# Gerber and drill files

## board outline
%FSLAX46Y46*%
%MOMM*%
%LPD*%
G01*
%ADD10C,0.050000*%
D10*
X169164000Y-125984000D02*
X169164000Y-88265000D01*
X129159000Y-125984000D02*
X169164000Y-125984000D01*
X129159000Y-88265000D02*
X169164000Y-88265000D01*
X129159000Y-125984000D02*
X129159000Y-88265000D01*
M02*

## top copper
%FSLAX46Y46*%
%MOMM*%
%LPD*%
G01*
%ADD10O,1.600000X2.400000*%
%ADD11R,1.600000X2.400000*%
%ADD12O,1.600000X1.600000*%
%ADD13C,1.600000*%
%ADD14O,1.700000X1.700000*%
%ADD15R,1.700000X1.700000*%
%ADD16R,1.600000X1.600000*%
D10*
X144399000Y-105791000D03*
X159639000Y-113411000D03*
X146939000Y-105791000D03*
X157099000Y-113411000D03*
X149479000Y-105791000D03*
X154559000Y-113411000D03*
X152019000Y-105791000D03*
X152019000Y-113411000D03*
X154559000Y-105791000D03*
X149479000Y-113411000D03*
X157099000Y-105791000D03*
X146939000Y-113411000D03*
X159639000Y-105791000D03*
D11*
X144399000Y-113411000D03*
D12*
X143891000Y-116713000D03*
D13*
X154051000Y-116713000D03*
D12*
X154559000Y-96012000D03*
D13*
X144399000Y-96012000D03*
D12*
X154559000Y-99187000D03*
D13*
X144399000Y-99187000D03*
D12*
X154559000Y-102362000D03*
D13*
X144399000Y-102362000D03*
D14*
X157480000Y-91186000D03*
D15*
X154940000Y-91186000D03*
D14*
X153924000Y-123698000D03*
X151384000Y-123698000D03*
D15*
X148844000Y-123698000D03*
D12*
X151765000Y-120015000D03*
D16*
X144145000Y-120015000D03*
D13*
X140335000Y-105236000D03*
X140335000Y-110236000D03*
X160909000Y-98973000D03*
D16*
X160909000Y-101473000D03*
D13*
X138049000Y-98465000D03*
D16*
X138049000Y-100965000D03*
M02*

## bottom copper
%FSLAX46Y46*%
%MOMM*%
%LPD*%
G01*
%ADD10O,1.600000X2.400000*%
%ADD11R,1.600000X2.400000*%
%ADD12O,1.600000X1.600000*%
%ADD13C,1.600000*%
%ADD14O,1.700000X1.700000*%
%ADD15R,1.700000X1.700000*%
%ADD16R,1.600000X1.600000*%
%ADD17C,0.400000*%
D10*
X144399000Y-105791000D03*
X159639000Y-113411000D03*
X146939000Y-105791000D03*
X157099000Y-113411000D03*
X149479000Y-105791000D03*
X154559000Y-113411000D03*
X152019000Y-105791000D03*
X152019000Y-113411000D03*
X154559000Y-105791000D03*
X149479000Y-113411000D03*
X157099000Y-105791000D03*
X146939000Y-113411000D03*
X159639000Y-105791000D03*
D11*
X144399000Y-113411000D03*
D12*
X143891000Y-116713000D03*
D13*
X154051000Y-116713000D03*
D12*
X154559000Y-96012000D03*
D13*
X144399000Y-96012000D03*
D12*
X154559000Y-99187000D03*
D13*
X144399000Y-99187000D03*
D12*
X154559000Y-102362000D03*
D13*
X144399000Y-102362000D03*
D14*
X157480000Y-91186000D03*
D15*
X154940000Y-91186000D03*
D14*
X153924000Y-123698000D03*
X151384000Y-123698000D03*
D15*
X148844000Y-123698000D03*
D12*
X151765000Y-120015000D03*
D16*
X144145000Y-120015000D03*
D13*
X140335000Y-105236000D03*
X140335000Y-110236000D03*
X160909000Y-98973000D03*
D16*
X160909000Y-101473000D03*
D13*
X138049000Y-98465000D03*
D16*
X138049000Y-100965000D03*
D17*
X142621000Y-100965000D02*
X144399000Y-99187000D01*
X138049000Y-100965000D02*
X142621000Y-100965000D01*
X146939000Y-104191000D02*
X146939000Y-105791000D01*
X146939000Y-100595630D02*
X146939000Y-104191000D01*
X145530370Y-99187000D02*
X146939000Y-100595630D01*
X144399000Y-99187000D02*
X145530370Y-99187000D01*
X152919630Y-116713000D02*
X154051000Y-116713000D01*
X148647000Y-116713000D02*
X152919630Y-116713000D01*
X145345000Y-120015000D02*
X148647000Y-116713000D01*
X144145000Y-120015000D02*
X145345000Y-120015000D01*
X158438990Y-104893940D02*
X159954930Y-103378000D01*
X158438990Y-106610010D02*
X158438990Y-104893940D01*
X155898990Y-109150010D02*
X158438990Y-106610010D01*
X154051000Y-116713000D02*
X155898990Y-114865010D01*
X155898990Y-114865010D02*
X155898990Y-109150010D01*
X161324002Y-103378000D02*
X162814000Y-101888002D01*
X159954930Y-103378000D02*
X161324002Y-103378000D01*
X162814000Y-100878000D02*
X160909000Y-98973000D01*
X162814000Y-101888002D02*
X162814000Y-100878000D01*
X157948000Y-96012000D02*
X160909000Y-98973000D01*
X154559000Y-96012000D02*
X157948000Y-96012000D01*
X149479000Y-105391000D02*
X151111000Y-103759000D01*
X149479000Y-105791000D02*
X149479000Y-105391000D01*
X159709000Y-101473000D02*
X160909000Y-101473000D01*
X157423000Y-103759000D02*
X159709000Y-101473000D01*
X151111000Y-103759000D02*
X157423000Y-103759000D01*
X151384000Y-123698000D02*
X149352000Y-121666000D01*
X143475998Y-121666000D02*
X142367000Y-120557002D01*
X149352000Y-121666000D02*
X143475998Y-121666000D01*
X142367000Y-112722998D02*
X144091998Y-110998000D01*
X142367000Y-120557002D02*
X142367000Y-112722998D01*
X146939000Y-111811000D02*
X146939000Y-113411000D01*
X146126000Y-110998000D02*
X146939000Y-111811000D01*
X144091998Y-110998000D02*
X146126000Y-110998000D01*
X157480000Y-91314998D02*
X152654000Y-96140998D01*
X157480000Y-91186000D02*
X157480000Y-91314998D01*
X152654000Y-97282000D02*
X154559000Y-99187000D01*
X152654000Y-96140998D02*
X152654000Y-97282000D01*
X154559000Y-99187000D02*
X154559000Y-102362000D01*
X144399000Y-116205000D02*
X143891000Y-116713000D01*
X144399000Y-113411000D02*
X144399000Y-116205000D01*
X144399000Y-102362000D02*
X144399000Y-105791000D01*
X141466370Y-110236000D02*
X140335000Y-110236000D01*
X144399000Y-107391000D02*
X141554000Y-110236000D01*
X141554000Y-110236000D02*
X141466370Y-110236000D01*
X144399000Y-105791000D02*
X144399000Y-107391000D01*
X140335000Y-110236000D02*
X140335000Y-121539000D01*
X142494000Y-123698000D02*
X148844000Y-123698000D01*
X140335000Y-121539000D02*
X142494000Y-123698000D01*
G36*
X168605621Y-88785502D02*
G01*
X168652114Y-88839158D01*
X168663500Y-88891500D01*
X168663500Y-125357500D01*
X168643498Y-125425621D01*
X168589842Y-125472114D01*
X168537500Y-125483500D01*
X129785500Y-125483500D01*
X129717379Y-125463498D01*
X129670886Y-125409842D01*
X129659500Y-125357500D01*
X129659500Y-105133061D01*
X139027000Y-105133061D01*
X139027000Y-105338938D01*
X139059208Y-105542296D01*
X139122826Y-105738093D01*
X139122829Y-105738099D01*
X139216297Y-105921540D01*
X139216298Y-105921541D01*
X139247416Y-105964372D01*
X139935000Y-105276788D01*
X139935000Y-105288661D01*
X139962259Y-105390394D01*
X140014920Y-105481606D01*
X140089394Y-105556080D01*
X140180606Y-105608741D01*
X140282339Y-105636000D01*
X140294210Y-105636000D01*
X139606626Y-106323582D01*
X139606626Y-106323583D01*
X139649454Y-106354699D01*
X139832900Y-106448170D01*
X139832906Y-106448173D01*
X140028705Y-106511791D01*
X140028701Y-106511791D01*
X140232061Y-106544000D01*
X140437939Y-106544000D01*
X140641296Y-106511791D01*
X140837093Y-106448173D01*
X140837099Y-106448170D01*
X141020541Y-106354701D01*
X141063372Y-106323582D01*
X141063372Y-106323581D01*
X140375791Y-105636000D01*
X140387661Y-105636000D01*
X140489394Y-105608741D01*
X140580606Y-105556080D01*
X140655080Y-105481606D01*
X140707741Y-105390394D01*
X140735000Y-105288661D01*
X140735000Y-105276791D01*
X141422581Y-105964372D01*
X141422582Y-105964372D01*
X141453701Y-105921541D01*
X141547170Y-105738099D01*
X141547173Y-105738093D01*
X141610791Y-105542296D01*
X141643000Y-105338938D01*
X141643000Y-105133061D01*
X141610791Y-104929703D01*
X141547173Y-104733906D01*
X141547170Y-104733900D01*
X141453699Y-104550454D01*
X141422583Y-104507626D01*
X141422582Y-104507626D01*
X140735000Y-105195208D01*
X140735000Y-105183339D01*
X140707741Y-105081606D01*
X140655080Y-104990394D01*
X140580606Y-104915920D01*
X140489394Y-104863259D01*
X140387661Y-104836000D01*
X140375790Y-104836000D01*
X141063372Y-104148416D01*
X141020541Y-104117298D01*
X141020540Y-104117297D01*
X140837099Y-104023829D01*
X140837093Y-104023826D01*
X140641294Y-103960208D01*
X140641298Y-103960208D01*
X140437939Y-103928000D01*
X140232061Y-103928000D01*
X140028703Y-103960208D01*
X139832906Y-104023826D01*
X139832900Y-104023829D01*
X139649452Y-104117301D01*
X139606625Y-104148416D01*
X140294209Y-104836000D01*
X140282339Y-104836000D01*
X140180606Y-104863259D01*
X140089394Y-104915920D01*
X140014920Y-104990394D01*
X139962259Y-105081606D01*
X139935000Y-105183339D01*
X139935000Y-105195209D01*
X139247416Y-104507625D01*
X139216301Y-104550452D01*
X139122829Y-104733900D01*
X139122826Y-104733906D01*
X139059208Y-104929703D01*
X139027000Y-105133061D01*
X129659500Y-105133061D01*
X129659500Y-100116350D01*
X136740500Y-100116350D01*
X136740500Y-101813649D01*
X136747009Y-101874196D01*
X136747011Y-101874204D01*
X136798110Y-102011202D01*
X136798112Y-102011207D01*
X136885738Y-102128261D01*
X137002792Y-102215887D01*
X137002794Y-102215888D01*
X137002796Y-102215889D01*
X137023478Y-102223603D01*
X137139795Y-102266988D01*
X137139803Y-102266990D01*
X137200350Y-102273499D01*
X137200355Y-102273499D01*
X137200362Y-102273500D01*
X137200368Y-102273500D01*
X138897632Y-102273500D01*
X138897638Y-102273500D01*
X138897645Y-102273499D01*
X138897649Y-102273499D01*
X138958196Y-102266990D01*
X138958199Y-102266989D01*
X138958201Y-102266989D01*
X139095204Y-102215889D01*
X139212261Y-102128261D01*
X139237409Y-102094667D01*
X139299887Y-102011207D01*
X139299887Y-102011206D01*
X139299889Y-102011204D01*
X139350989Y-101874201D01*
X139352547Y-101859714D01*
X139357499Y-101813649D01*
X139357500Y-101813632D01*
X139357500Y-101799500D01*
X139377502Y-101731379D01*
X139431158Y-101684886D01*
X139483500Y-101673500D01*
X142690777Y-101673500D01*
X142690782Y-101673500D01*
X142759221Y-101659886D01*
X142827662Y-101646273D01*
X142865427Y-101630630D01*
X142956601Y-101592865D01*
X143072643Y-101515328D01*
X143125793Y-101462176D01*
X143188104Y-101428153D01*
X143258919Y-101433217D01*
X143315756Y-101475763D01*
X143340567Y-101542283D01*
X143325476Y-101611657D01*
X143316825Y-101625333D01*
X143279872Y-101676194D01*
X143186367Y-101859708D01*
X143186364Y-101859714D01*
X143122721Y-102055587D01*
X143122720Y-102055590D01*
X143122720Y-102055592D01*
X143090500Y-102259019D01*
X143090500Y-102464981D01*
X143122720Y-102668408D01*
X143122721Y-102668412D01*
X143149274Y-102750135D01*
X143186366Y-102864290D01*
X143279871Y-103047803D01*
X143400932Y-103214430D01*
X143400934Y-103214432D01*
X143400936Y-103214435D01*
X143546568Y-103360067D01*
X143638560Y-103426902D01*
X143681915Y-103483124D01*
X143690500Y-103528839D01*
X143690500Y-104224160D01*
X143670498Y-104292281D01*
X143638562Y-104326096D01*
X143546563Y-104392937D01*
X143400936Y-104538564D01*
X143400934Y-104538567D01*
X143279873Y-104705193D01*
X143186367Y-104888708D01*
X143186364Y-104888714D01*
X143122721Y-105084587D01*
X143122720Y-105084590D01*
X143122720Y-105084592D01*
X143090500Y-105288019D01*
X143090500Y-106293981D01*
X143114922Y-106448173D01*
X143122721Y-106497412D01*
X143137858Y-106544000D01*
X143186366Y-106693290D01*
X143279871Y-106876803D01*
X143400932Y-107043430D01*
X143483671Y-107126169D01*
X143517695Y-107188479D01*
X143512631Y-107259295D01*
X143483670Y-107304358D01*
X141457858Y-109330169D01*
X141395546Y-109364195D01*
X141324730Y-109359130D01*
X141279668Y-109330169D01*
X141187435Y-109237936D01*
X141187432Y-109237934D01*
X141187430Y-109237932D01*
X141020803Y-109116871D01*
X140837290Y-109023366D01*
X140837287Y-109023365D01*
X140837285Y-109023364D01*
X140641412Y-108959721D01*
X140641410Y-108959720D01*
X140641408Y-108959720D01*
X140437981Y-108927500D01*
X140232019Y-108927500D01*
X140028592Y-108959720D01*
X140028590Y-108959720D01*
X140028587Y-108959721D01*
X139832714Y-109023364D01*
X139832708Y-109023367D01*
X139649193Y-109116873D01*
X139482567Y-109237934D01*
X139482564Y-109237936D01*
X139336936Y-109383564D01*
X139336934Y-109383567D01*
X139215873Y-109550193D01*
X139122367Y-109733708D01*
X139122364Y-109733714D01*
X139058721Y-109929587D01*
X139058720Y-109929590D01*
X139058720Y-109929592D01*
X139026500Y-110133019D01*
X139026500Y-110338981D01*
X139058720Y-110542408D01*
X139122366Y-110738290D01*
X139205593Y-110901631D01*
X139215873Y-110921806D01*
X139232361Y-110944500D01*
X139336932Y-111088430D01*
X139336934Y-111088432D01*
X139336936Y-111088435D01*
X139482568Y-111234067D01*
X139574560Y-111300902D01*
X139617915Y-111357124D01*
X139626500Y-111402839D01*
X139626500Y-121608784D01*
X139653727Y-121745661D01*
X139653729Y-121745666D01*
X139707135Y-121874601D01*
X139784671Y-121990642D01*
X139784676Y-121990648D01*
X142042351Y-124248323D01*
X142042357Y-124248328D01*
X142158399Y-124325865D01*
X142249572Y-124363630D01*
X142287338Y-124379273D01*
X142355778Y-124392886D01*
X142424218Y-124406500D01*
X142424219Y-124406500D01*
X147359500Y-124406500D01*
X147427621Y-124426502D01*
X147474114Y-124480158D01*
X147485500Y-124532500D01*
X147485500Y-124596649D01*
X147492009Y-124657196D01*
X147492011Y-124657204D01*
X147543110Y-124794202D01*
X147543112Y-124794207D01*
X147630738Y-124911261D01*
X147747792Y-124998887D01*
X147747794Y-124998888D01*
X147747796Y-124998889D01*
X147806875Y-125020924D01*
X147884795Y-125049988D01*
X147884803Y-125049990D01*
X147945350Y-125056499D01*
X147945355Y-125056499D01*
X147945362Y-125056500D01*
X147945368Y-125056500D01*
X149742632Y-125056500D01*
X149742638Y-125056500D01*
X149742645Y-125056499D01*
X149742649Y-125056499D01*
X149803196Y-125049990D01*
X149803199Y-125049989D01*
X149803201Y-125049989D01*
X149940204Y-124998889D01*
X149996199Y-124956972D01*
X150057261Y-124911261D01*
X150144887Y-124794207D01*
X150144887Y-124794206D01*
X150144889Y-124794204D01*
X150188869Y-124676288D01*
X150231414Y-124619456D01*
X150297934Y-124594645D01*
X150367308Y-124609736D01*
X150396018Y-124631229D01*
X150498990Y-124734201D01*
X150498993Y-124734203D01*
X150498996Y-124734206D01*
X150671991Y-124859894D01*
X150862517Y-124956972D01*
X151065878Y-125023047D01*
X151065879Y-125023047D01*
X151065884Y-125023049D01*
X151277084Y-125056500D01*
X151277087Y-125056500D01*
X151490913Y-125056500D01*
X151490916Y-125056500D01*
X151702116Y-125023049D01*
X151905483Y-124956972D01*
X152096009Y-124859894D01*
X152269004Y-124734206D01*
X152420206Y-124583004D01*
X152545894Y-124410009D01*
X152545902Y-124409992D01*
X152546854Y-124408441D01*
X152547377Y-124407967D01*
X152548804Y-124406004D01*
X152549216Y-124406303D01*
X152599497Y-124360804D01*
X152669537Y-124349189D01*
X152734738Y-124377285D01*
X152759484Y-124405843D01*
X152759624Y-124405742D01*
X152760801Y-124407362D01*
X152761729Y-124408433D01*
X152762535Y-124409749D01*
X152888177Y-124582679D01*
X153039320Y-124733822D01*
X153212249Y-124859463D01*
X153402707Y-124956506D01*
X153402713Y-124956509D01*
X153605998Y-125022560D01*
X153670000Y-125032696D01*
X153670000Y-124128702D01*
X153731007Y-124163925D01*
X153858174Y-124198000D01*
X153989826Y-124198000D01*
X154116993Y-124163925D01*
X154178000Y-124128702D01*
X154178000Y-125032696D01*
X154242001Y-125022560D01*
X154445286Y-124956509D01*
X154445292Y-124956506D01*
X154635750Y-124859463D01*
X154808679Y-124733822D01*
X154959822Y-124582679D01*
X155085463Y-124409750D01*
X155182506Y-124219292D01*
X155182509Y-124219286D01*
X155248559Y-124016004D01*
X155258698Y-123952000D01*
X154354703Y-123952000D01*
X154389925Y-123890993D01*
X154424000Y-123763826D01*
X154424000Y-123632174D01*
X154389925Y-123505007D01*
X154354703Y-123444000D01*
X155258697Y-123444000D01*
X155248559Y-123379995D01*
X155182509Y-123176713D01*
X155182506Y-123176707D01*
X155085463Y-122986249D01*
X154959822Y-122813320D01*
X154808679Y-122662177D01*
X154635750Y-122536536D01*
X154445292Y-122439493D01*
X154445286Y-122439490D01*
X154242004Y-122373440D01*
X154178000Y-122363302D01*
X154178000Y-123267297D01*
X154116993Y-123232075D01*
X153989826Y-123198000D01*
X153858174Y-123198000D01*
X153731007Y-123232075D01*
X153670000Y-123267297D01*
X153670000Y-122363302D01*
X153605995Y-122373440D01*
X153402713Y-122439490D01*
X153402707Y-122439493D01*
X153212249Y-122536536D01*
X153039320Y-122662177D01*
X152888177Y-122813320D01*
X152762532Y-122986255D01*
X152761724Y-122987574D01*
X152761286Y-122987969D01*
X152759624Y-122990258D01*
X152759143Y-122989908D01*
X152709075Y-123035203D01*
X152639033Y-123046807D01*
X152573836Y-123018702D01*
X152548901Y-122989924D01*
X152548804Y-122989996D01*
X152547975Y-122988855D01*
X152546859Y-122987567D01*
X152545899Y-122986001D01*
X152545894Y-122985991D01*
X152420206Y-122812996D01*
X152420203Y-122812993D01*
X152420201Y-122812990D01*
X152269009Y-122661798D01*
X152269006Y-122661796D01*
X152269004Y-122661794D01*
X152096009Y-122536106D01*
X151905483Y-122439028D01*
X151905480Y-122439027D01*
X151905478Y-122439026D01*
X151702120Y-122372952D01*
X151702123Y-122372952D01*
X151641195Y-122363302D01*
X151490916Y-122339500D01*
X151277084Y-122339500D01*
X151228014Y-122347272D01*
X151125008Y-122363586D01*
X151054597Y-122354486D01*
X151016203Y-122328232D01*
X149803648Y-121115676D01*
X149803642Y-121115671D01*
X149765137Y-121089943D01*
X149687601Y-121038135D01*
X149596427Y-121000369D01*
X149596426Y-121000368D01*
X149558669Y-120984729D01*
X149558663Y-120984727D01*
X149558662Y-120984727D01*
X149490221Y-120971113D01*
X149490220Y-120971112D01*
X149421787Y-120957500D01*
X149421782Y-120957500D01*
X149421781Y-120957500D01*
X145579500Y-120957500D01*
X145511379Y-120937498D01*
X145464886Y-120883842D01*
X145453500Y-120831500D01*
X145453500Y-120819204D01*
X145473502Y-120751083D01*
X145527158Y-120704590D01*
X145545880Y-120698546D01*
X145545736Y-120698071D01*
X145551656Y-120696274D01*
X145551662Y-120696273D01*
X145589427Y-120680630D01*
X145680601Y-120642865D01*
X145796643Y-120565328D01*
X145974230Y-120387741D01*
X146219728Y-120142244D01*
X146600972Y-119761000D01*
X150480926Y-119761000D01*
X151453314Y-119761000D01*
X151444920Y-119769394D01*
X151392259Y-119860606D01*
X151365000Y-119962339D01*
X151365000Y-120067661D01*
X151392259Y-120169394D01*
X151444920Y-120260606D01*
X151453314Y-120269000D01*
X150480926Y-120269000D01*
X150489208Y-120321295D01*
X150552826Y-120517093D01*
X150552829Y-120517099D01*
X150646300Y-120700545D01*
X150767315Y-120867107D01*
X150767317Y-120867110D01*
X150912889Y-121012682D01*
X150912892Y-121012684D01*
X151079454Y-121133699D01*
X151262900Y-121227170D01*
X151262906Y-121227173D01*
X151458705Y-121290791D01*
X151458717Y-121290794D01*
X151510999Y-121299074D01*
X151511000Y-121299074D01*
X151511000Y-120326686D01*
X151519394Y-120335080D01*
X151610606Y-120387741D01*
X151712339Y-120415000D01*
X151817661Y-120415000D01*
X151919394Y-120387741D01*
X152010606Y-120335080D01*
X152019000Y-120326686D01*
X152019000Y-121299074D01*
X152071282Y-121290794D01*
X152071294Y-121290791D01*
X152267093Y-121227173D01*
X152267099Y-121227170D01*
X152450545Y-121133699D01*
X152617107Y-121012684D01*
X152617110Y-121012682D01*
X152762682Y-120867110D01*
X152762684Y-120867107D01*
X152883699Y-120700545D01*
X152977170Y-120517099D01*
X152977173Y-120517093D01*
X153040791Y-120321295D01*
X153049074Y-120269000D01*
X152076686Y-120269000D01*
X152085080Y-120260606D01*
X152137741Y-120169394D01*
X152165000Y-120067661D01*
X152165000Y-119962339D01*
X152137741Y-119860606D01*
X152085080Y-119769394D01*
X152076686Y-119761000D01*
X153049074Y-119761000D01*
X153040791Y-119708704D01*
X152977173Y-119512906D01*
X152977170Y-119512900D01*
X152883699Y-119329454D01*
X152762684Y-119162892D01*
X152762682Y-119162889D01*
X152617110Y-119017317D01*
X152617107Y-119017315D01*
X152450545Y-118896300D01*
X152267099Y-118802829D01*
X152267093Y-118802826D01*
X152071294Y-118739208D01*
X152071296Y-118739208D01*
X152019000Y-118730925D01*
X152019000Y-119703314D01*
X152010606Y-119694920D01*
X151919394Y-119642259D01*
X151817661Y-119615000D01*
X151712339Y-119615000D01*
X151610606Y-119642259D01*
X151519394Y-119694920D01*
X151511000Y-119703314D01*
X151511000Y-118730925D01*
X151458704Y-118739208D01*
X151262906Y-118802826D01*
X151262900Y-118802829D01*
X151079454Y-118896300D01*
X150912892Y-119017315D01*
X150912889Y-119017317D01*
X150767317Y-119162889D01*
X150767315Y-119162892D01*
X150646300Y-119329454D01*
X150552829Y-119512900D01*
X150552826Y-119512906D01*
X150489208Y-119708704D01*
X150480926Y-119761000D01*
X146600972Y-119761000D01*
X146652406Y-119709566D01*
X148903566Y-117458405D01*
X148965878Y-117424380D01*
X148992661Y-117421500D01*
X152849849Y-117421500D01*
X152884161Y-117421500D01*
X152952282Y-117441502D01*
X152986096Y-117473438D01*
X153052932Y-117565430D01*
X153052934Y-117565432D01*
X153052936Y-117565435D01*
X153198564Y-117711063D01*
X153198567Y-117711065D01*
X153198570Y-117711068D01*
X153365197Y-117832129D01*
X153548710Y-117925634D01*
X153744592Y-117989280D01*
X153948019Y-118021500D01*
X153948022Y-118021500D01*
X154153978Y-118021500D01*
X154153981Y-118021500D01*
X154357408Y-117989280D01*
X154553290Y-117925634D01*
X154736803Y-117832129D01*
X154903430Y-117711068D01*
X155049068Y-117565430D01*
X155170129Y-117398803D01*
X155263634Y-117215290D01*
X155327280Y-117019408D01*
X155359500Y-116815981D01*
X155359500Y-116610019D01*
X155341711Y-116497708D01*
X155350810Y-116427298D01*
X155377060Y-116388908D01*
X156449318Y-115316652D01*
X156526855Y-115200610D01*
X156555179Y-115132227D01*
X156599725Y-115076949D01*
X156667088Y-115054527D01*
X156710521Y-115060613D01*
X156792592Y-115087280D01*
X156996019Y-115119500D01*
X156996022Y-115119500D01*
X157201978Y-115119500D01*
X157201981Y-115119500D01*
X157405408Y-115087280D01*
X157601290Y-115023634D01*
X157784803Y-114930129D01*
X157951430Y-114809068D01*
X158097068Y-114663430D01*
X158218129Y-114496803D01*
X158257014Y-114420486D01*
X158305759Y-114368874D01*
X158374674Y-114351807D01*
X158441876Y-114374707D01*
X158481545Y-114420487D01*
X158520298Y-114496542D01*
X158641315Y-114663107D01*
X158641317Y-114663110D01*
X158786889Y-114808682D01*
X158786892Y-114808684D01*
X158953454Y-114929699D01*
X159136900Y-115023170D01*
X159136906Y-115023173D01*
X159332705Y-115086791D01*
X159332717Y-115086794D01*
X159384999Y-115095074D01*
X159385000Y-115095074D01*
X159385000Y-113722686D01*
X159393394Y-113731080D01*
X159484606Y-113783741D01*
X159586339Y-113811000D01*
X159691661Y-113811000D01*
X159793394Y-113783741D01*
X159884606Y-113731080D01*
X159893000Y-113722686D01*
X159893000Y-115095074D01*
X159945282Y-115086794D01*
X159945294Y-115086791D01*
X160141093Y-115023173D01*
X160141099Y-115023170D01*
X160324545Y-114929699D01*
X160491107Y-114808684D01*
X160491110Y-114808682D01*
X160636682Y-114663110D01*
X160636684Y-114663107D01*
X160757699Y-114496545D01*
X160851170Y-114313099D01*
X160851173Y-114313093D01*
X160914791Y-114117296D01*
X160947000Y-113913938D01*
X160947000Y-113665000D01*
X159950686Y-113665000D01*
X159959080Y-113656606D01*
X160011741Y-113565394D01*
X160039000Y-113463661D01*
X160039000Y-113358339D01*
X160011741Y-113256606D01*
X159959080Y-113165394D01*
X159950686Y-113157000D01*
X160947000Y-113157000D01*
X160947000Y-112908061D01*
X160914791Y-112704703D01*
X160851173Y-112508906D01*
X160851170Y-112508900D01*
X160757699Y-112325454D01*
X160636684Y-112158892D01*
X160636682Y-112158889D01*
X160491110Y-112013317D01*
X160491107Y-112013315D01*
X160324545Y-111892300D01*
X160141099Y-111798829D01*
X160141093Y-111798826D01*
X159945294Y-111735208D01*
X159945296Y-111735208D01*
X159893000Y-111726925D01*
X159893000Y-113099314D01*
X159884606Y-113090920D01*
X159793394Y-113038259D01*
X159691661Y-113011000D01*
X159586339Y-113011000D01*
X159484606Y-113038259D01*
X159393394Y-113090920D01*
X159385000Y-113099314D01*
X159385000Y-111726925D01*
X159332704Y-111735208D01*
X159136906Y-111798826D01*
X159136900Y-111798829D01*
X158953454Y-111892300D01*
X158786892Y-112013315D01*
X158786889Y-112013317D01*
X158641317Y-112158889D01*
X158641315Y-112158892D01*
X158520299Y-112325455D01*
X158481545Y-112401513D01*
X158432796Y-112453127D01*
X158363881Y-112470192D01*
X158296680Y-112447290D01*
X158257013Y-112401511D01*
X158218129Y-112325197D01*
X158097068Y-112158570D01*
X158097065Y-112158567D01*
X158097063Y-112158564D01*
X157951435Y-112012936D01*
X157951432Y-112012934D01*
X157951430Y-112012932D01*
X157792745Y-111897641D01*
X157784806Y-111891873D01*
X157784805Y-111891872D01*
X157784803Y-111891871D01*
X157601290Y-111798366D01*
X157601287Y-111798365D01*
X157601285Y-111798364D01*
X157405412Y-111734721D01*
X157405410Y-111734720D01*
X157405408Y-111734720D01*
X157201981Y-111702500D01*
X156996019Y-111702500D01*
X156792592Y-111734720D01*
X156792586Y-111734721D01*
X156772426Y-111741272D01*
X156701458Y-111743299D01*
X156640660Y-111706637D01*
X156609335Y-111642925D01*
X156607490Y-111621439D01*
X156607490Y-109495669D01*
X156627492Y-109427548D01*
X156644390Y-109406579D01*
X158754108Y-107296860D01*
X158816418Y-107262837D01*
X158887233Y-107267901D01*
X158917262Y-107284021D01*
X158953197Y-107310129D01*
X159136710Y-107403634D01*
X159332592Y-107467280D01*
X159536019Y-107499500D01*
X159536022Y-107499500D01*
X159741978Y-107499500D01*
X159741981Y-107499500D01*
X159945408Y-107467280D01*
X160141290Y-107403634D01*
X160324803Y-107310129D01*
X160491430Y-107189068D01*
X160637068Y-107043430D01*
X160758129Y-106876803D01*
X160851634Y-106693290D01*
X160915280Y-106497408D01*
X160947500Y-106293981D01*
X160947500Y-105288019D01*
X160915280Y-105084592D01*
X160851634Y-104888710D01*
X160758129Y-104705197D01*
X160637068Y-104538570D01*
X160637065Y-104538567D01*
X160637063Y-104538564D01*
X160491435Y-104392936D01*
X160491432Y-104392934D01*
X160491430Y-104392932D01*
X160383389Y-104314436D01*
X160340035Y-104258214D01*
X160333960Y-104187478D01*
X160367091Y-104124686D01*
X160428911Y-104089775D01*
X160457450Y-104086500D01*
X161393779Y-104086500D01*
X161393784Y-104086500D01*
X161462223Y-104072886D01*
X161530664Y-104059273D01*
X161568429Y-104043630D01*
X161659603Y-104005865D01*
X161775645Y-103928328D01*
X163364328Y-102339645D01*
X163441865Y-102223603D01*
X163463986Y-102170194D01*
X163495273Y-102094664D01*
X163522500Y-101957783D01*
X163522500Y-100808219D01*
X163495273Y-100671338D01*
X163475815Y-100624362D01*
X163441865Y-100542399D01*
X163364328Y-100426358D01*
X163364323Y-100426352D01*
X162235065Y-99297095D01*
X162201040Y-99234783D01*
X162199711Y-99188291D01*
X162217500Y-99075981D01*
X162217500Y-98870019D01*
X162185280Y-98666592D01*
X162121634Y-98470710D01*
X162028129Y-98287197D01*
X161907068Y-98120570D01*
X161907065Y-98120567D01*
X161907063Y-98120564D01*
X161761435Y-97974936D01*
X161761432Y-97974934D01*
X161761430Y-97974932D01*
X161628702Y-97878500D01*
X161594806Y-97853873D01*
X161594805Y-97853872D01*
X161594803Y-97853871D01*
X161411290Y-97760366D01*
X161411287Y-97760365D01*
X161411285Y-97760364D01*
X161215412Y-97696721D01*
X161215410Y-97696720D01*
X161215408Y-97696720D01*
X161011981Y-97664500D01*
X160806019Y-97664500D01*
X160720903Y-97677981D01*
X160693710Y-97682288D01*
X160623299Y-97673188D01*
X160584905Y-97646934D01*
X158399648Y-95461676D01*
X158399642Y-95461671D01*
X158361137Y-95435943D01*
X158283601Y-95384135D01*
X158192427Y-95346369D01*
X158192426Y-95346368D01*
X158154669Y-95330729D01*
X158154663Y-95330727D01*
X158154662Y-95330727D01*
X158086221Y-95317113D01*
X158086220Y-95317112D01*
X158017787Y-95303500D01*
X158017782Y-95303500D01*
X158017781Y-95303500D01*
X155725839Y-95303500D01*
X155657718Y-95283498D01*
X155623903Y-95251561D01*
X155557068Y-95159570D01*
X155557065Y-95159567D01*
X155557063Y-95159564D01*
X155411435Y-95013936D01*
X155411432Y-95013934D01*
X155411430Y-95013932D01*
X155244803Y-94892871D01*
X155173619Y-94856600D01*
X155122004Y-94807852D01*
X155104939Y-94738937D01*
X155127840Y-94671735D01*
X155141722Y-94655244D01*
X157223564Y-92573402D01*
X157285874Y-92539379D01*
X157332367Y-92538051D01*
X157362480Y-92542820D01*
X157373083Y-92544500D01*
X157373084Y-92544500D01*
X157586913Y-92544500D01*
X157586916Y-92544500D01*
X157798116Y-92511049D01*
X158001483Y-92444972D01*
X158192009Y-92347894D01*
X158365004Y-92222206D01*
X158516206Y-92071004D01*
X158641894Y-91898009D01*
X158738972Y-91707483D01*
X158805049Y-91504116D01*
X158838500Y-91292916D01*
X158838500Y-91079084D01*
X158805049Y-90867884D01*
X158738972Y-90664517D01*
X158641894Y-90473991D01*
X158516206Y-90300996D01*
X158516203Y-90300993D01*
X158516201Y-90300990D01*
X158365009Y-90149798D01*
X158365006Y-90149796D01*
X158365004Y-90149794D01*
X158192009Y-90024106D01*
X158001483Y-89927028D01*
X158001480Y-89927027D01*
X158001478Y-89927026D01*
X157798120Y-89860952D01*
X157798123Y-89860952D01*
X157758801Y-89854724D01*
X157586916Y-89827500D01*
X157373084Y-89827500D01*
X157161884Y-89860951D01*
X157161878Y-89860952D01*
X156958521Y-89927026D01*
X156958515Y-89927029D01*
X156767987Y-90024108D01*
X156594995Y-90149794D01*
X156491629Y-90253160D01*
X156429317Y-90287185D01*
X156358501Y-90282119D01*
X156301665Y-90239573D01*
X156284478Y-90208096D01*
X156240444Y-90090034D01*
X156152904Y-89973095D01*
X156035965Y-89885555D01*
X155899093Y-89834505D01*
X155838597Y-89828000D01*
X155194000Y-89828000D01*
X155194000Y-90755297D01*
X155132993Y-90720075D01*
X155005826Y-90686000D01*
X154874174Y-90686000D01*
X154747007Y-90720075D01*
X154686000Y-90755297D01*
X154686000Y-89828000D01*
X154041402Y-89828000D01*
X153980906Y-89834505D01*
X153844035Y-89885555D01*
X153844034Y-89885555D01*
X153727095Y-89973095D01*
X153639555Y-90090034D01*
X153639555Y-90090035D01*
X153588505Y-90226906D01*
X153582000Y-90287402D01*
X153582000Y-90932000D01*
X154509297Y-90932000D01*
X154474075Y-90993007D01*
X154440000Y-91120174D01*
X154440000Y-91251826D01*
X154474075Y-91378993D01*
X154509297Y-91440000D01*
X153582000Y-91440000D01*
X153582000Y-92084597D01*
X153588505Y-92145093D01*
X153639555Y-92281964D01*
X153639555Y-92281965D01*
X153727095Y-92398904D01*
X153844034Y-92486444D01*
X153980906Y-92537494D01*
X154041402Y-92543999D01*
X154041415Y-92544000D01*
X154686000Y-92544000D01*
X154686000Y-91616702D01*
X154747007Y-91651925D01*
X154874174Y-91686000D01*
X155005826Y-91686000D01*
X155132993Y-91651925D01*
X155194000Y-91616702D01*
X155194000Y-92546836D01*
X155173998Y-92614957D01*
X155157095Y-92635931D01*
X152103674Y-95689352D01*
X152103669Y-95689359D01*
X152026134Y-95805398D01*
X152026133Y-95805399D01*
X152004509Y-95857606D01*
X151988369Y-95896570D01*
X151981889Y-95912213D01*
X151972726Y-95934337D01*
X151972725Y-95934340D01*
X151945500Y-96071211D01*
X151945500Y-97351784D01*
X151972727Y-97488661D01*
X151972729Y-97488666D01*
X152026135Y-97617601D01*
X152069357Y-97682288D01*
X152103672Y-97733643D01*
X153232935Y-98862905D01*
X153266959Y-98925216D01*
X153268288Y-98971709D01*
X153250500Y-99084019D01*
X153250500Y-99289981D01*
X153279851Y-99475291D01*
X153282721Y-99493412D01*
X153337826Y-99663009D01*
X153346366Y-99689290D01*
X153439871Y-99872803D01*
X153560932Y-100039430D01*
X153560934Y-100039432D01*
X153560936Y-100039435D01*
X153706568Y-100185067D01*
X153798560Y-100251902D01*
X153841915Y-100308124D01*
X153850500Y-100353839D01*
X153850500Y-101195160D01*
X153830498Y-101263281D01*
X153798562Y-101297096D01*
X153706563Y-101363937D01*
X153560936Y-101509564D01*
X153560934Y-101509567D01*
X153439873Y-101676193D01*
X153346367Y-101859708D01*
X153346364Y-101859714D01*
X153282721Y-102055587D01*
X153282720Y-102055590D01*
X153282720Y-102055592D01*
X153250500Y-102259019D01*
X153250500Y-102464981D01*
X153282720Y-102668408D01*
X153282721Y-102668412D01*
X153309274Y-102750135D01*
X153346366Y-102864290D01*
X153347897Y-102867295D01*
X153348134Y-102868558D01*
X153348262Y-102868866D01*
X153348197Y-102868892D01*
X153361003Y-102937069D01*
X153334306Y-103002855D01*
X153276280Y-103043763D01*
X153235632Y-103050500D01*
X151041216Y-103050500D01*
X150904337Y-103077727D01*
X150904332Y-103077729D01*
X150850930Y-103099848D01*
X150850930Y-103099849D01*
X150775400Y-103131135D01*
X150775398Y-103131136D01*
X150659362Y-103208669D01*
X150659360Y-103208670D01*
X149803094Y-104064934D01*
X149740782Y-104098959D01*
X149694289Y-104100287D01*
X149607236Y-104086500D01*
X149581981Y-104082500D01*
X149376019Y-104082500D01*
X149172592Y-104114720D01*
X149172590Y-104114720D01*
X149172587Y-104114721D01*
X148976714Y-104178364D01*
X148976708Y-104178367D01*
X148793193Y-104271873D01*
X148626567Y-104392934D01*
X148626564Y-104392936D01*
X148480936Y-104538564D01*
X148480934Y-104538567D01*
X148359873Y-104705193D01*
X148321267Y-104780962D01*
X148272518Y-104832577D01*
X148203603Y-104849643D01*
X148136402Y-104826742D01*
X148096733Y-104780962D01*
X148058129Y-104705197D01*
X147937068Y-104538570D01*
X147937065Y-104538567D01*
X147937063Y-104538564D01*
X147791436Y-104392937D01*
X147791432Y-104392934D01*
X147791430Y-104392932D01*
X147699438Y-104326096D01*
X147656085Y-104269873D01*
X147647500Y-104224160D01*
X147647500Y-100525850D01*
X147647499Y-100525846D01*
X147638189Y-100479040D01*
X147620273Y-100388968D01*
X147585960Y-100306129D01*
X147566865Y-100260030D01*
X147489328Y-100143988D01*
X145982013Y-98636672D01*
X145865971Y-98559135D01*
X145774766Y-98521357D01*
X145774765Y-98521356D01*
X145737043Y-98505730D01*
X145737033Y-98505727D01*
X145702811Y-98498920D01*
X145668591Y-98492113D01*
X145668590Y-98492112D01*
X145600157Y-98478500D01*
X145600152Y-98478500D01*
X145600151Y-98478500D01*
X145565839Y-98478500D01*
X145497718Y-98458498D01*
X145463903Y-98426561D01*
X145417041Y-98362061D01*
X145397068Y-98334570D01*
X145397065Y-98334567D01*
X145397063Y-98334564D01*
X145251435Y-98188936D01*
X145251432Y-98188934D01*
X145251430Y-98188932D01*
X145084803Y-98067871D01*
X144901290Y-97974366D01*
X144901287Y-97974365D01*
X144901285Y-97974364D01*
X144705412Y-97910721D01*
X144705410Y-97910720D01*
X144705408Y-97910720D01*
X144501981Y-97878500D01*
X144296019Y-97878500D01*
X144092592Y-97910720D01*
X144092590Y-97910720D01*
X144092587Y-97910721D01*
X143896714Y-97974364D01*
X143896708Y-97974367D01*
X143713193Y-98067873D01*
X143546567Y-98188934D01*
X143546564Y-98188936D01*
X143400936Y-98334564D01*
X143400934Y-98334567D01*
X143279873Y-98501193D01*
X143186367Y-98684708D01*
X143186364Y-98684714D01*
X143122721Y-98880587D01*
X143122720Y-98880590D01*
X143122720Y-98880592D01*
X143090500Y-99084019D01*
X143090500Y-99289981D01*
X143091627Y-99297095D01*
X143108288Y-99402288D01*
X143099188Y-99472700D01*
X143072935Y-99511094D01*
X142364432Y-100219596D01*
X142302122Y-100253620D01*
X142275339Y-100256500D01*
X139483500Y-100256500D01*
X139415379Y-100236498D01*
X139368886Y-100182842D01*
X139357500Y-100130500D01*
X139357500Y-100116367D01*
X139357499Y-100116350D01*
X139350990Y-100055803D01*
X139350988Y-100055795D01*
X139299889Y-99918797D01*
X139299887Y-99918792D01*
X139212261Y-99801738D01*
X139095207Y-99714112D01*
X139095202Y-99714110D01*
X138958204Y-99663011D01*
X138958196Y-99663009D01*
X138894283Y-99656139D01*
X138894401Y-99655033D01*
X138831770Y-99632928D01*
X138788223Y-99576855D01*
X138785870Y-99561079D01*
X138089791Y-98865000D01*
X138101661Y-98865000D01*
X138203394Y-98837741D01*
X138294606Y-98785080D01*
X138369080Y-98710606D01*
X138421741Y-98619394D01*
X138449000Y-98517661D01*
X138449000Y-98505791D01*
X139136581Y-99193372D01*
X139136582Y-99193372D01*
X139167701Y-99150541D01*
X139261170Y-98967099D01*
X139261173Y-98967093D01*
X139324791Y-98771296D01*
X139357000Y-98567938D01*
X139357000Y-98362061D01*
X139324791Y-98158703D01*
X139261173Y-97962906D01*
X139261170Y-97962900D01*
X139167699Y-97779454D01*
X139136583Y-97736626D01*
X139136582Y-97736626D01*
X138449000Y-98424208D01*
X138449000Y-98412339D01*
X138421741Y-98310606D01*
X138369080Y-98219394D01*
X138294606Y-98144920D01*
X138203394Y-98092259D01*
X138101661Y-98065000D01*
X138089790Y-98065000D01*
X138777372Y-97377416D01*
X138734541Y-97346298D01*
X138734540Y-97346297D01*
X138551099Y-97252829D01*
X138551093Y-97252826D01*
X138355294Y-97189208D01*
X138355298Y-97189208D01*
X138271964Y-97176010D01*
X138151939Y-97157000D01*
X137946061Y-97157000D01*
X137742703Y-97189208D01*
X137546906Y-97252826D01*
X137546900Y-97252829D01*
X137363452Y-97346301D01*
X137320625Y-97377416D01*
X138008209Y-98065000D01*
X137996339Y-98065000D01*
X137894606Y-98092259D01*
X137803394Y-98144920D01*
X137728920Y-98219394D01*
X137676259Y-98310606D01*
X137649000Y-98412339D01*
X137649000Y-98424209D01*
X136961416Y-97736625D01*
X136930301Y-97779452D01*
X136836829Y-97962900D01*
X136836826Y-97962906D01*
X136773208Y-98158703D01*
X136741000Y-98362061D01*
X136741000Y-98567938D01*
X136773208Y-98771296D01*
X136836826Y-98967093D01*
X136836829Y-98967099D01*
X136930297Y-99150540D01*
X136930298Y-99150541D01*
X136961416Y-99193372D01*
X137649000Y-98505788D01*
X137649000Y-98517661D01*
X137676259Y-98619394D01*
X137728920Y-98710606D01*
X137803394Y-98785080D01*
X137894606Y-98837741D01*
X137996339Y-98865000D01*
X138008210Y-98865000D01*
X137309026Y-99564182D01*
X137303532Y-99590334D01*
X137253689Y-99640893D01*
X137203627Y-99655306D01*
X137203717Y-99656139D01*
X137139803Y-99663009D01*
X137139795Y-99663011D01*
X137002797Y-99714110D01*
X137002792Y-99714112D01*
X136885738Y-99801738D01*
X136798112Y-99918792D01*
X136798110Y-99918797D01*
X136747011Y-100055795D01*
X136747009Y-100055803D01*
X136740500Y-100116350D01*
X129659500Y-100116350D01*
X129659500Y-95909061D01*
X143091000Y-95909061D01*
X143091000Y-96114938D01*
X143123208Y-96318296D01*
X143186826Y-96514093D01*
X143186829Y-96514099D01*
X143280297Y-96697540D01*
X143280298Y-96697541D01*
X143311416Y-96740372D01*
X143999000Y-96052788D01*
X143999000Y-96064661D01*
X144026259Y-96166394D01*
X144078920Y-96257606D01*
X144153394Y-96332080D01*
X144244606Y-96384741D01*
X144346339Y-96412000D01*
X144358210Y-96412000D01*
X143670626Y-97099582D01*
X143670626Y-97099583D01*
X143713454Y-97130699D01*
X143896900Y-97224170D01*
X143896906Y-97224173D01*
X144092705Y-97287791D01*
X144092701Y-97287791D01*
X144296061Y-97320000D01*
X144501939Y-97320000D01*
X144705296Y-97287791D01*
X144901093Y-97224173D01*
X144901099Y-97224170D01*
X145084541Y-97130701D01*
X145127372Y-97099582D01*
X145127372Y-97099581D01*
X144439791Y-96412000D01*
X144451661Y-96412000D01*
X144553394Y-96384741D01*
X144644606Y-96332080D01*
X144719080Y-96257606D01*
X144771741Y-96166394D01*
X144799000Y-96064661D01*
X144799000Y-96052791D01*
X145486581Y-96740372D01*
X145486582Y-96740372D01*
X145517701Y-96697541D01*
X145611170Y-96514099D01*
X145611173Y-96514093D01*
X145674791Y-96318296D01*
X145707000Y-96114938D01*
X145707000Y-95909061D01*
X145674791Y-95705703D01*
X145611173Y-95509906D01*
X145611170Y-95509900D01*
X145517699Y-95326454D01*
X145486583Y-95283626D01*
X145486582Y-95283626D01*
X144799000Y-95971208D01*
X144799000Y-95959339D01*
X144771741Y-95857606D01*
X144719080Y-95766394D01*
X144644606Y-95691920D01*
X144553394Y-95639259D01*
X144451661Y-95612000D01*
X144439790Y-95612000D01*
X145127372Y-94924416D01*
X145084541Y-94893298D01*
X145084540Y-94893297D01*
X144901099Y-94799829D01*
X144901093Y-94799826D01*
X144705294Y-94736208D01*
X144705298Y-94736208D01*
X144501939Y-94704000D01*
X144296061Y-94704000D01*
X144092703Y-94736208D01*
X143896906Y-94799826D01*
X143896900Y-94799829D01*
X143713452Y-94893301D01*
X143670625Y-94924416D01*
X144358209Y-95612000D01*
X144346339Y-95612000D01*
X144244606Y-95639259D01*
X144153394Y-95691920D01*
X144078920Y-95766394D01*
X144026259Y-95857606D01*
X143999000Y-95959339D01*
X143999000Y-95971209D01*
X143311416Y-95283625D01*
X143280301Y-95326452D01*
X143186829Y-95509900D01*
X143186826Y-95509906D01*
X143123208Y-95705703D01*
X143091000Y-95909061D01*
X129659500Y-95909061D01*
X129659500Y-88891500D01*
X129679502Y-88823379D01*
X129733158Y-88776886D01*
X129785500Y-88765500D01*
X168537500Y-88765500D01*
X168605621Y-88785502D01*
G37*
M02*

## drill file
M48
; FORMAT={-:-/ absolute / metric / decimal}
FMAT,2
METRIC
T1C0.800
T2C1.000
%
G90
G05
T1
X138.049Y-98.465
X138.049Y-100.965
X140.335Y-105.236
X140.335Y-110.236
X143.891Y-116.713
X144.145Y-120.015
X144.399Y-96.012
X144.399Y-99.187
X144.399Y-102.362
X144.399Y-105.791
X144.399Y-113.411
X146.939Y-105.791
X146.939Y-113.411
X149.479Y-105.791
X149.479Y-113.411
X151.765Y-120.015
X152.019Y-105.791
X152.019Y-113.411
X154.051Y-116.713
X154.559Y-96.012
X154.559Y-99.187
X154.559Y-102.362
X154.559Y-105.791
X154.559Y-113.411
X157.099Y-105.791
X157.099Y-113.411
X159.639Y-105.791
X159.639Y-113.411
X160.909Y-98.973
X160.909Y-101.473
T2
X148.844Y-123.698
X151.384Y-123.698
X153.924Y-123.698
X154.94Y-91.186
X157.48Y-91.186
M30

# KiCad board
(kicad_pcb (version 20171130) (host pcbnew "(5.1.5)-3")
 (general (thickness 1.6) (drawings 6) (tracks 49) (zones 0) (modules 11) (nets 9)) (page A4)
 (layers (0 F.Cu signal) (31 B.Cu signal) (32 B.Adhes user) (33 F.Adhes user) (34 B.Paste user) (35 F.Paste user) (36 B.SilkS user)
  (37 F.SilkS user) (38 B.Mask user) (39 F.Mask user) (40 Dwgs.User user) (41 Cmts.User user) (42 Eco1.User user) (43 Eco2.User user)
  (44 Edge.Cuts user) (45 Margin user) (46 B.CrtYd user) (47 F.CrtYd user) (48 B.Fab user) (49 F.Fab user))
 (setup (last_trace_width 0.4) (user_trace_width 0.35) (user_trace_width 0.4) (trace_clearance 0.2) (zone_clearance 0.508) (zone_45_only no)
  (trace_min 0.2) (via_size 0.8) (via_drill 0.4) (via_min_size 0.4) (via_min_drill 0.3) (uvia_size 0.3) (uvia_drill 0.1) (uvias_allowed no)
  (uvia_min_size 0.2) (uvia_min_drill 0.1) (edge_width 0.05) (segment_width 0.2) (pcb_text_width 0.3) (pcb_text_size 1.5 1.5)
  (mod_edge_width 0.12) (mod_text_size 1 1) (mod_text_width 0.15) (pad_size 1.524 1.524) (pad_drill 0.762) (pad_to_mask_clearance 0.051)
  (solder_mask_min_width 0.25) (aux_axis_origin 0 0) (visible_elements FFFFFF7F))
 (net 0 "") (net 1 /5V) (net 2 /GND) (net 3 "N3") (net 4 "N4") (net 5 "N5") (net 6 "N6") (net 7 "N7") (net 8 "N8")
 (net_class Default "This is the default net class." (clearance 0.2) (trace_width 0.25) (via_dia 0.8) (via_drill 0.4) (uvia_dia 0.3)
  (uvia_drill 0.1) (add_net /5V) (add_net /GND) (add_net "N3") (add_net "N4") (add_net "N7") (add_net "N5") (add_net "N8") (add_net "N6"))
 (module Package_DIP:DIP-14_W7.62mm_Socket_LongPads (layer F.Cu) (at 144.399 113.411 90)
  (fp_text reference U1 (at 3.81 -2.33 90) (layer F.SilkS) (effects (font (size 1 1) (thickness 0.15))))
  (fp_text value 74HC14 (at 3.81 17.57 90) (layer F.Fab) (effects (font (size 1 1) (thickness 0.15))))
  (pad 14 thru_hole oval (at 7.62 0 90) (size 2.4 1.6) (drill 0.8) (layers *.Cu *.Mask) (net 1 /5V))
  (pad 7 thru_hole oval (at 0 15.24 90) (size 2.4 1.6) (drill 0.8) (layers *.Cu *.Mask) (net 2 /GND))
  (pad 13 thru_hole oval (at 7.62 2.54 90) (size 2.4 1.6) (drill 0.8) (layers *.Cu *.Mask) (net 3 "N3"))
  (pad 6 thru_hole oval (at 0 12.7 90) (size 2.4 1.6) (drill 0.8) (layers *.Cu *.Mask))
  (pad 12 thru_hole oval (at 7.62 5.08 90) (size 2.4 1.6) (drill 0.8) (layers *.Cu *.Mask) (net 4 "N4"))
  (pad 5 thru_hole oval (at 0 10.16 90) (size 2.4 1.6) (drill 0.8) (layers *.Cu *.Mask))
  (pad 11 thru_hole oval (at 7.62 7.62 90) (size 2.4 1.6) (drill 0.8) (layers *.Cu *.Mask))
  (pad 4 thru_hole oval (at 0 7.62 90) (size 2.4 1.6) (drill 0.8) (layers *.Cu *.Mask))
  (pad 10 thru_hole oval (at 7.62 10.16 90) (size 2.4 1.6) (drill 0.8) (layers *.Cu *.Mask))
  (pad 3 thru_hole oval (at 0 5.08 90) (size 2.4 1.6) (drill 0.8) (layers *.Cu *.Mask))
  (pad 9 thru_hole oval (at 7.62 12.7 90) (size 2.4 1.6) (drill 0.8) (layers *.Cu *.Mask))
  (pad 2 thru_hole oval (at 0 2.54 90) (size 2.4 1.6) (drill 0.8) (layers *.Cu *.Mask) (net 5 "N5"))
  (pad 8 thru_hole oval (at 7.62 15.24 90) (size 2.4 1.6) (drill 0.8) (layers *.Cu *.Mask))
  (pad 1 thru_hole rect (at 0 0 90) (size 2.4 1.6) (drill 0.8) (layers *.Cu *.Mask) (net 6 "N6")))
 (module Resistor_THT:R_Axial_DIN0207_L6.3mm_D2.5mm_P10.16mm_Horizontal (layer F.Cu) (at 154.051 116.713 180)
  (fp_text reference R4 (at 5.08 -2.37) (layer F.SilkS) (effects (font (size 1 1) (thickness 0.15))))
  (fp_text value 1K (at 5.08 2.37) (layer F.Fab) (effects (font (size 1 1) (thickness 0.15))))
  (pad 2 thru_hole oval (at 10.16 0 180) (size 1.6 1.6) (drill 0.8) (layers *.Cu *.Mask) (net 6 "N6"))
  (pad 1 thru_hole circle (at 0 0 180) (size 1.6 1.6) (drill 0.8) (layers *.Cu *.Mask) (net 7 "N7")))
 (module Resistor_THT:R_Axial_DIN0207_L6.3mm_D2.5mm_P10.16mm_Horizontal (layer F.Cu) (at 144.399 96.012)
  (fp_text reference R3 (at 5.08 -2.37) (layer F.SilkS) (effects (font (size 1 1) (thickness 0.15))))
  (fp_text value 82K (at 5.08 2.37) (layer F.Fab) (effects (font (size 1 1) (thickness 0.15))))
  (pad 2 thru_hole oval (at 10.16 0) (size 1.6 1.6) (drill 0.8) (layers *.Cu *.Mask) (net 7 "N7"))
  (pad 1 thru_hole circle (at 0 0) (size 1.6 1.6) (drill 0.8) (layers *.Cu *.Mask) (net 2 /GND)))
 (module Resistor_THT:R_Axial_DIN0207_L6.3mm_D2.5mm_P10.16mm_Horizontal (layer F.Cu) (at 144.399 99.187)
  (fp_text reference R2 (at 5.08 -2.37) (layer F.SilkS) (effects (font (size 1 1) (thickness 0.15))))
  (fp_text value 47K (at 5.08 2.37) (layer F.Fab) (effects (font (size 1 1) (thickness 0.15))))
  (pad 2 thru_hole oval (at 10.16 0) (size 1.6 1.6) (drill 0.8) (layers *.Cu *.Mask) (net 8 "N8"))
  (pad 1 thru_hole circle (at 0 0) (size 1.6 1.6) (drill 0.8) (layers *.Cu *.Mask) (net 3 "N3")))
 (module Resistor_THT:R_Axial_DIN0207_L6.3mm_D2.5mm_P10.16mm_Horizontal (layer F.Cu) (at 144.399 102.362)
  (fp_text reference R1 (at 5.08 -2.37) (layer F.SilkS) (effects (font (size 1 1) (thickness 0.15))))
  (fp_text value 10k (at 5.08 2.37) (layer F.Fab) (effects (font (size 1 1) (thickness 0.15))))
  (pad 2 thru_hole oval (at 10.16 0) (size 1.6 1.6) (drill 0.8) (layers *.Cu *.Mask) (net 8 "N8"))
  (pad 1 thru_hole circle (at 0 0) (size 1.6 1.6) (drill 0.8) (layers *.Cu *.Mask) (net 1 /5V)))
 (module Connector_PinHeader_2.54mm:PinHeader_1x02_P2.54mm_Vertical (layer F.Cu) (at 154.94 91.186 90)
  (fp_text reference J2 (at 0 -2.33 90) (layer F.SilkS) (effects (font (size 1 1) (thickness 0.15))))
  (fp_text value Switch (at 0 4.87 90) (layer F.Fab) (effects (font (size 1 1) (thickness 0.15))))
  (pad 2 thru_hole oval (at 0 2.54 90) (size 1.7 1.7) (drill 1) (layers *.Cu *.Mask) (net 8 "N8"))
  (pad 1 thru_hole rect (at 0 0 90) (size 1.7 1.7) (drill 1) (layers *.Cu *.Mask) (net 2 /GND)))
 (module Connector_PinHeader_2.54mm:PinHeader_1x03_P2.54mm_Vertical (layer F.Cu) (at 148.844 123.698 90)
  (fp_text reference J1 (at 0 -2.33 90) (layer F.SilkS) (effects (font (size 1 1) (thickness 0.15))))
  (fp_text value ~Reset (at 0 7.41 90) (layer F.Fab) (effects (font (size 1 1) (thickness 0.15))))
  (pad 3 thru_hole oval (at 0 5.08 90) (size 1.7 1.7) (drill 1) (layers *.Cu *.Mask) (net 2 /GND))
  (pad 2 thru_hole oval (at 0 2.54 90) (size 1.7 1.7) (drill 1) (layers *.Cu *.Mask) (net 5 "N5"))
  (pad 1 thru_hole rect (at 0 0 90) (size 1.7 1.7) (drill 1) (layers *.Cu *.Mask) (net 1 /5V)))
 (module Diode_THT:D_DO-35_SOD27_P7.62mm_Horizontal (layer F.Cu) (at 144.145 120.015)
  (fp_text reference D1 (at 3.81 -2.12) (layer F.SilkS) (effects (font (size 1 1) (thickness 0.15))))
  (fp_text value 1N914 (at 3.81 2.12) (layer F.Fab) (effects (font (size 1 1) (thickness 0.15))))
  (pad 2 thru_hole oval (at 7.62 0) (size 1.6 1.6) (drill 0.8) (layers *.Cu *.Mask) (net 2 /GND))
  (pad 1 thru_hole rect (at 0 0) (size 1.6 1.6) (drill 0.8) (layers *.Cu *.Mask) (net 7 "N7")))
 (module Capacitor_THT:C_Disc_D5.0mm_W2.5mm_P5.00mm (layer F.Cu) (at 140.335 110.236 90)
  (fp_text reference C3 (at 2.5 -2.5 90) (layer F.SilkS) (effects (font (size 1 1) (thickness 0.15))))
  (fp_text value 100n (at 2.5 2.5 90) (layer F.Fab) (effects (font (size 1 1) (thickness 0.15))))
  (pad 2 thru_hole circle (at 5 0 90) (size 1.6 1.6) (drill 0.8) (layers *.Cu *.Mask) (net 2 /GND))
  (pad 1 thru_hole circle (at 0 0 90) (size 1.6 1.6) (drill 0.8) (layers *.Cu *.Mask) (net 1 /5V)))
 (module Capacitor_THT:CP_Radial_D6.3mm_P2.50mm (layer F.Cu) (at 160.909 101.473 90)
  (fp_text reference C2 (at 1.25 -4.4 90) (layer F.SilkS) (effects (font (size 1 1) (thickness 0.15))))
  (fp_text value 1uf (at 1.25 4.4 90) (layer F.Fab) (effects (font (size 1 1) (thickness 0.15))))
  (pad 2 thru_hole circle (at 2.5 0 90) (size 1.6 1.6) (drill 0.8) (layers *.Cu *.Mask) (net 7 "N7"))
  (pad 1 thru_hole rect (at 0 0 90) (size 1.6 1.6) (drill 0.8) (layers *.Cu *.Mask) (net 4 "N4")))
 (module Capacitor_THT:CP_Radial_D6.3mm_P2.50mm (layer F.Cu) (at 138.049 100.965 90)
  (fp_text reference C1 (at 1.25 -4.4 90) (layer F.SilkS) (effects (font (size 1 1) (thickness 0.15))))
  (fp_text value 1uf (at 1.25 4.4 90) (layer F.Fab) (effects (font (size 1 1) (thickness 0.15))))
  (pad 2 thru_hole circle (at 2.5 0 90) (size 1.6 1.6) (drill 0.8) (layers *.Cu *.Mask) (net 2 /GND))
  (pad 1 thru_hole rect (at 0 0 90) (size 1.6 1.6) (drill 0.8) (layers *.Cu *.Mask) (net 3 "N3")))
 (gr_line (start 169.164 125.984) (end 169.164 88.265) (layer Edge.Cuts) (width 0.05))
 (gr_line (start 129.159 125.984) (end 169.164 125.984) (layer Edge.Cuts) (width 0.05))
 (gr_line (start 129.159 88.265) (end 169.164 88.265) (layer Edge.Cuts) (width 0.05))
 (gr_line (start 129.159 125.984) (end 129.159 88.265) (layer Edge.Cuts) (width 0.05))
 (segment (start 142.621 100.965) (end 144.399 99.187) (width 0.4) (layer B.Cu) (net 3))
 (segment (start 138.049 100.965) (end 142.621 100.965) (width 0.4) (layer B.Cu) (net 3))
 (segment (start 146.939 104.191) (end 146.939 105.791) (width 0.4) (layer B.Cu) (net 3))
 (segment (start 146.939 100.59563) (end 146.939 104.191) (width 0.4) (layer B.Cu) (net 3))
 (segment (start 145.53037 99.187) (end 146.939 100.59563) (width 0.4) (layer B.Cu) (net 3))
 (segment (start 144.399 99.187) (end 145.53037 99.187) (width 0.4) (layer B.Cu) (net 3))
 (segment (start 152.91963 116.713) (end 154.051 116.713) (width 0.4) (layer B.Cu) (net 7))
 (segment (start 148.647 116.713) (end 152.91963 116.713) (width 0.4) (layer B.Cu) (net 7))
 (segment (start 145.345 120.015) (end 148.647 116.713) (width 0.4) (layer B.Cu) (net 7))
 (segment (start 144.145 120.015) (end 145.345 120.015) (width 0.4) (layer B.Cu) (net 7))
 (segment (start 158.43899 104.89394) (end 159.95493 103.378) (width 0.4) (layer B.Cu) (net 7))
 (segment (start 158.43899 106.61001) (end 158.43899 104.89394) (width 0.4) (layer B.Cu) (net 7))
 (segment (start 155.89899 109.15001) (end 158.43899 106.61001) (width 0.4) (layer B.Cu) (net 7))
 (segment (start 154.051 116.713) (end 155.89899 114.86501) (width 0.4) (layer B.Cu) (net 7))
 (segment (start 155.89899 114.86501) (end 155.89899 109.15001) (width 0.4) (layer B.Cu) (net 7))
 (segment (start 161.324002 103.378) (end 162.814 101.888002) (width 0.4) (layer B.Cu) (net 7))
 (segment (start 159.95493 103.378) (end 161.324002 103.378) (width 0.4) (layer B.Cu) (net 7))
 (segment (start 162.814 100.878) (end 160.909 98.973) (width 0.4) (layer B.Cu) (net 7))
 (segment (start 162.814 101.888002) (end 162.814 100.878) (width 0.4) (layer B.Cu) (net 7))
 (segment (start 157.948 96.012) (end 160.909 98.973) (width 0.4) (layer B.Cu) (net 7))
 (segment (start 154.559 96.012) (end 157.948 96.012) (width 0.4) (layer B.Cu) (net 7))
 (segment (start 149.479 105.391) (end 151.111 103.759) (width 0.4) (layer B.Cu) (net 4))
 (segment (start 149.479 105.791) (end 149.479 105.391) (width 0.4) (layer B.Cu) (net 4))
 (segment (start 159.709 101.473) (end 160.909 101.473) (width 0.4) (layer B.Cu) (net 4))
 (segment (start 157.423 103.759) (end 159.709 101.473) (width 0.4) (layer B.Cu) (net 4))
 (segment (start 151.111 103.759) (end 157.423 103.759) (width 0.4) (layer B.Cu) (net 4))
 (segment (start 151.384 123.698) (end 149.352 121.666) (width 0.4) (layer B.Cu) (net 5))
 (segment (start 143.475998 121.666) (end 142.367 120.557002) (width 0.4) (layer B.Cu) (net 5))
 (segment (start 149.352 121.666) (end 143.475998 121.666) (width 0.4) (layer B.Cu) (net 5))
 (segment (start 142.367 112.722998) (end 144.091998 110.998) (width 0.4) (layer B.Cu) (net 5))
 (segment (start 142.367 120.557002) (end 142.367 112.722998) (width 0.4) (layer B.Cu) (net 5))
 (segment (start 146.939 111.811) (end 146.939 113.411) (width 0.4) (layer B.Cu) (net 5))
 (segment (start 146.126 110.998) (end 146.939 111.811) (width 0.4) (layer B.Cu) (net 5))
 (segment (start 144.091998 110.998) (end 146.126 110.998) (width 0.4) (layer B.Cu) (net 5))
 (segment (start 157.48 91.314998) (end 152.654 96.140998) (width 0.4) (layer B.Cu) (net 8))
 (segment (start 157.48 91.186) (end 157.48 91.314998) (width 0.4) (layer B.Cu) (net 8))
 (segment (start 152.654 97.282) (end 154.559 99.187) (width 0.4) (layer B.Cu) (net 8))
 (segment (start 152.654 96.140998) (end 152.654 97.282) (width 0.4) (layer B.Cu) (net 8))
 (segment (start 154.559 99.187) (end 154.559 102.362) (width 0.4) (layer B.Cu) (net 8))
 (segment (start 144.399 116.205) (end 143.891 116.713) (width 0.4) (layer B.Cu) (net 6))
 (segment (start 144.399 113.411) (end 144.399 116.205) (width 0.4) (layer B.Cu) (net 6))
 (segment (start 144.399 102.362) (end 144.399 105.791) (width 0.4) (layer B.Cu) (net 1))
 (segment (start 141.46637 110.236) (end 140.335 110.236) (width 0.4) (layer B.Cu) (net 1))
 (segment (start 144.399 107.391) (end 141.554 110.236) (width 0.4) (layer B.Cu) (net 1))
 (segment (start 141.554 110.236) (end 141.46637 110.236) (width 0.4) (layer B.Cu) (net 1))
 (segment (start 144.399 105.791) (end 144.399 107.391) (width 0.4) (layer B.Cu) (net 1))
 (segment (start 140.335 110.236) (end 140.335 121.539) (width 0.4) (layer B.Cu) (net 1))
 (segment (start 142.494 123.698) (end 148.844 123.698) (width 0.4) (layer B.Cu) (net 1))
 (segment (start 140.335 121.539) (end 142.494 123.698) (width 0.4) (layer B.Cu) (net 1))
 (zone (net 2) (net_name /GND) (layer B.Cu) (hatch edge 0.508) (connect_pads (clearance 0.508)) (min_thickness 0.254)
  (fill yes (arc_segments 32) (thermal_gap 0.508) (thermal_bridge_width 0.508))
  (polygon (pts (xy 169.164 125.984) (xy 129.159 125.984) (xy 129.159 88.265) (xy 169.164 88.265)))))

